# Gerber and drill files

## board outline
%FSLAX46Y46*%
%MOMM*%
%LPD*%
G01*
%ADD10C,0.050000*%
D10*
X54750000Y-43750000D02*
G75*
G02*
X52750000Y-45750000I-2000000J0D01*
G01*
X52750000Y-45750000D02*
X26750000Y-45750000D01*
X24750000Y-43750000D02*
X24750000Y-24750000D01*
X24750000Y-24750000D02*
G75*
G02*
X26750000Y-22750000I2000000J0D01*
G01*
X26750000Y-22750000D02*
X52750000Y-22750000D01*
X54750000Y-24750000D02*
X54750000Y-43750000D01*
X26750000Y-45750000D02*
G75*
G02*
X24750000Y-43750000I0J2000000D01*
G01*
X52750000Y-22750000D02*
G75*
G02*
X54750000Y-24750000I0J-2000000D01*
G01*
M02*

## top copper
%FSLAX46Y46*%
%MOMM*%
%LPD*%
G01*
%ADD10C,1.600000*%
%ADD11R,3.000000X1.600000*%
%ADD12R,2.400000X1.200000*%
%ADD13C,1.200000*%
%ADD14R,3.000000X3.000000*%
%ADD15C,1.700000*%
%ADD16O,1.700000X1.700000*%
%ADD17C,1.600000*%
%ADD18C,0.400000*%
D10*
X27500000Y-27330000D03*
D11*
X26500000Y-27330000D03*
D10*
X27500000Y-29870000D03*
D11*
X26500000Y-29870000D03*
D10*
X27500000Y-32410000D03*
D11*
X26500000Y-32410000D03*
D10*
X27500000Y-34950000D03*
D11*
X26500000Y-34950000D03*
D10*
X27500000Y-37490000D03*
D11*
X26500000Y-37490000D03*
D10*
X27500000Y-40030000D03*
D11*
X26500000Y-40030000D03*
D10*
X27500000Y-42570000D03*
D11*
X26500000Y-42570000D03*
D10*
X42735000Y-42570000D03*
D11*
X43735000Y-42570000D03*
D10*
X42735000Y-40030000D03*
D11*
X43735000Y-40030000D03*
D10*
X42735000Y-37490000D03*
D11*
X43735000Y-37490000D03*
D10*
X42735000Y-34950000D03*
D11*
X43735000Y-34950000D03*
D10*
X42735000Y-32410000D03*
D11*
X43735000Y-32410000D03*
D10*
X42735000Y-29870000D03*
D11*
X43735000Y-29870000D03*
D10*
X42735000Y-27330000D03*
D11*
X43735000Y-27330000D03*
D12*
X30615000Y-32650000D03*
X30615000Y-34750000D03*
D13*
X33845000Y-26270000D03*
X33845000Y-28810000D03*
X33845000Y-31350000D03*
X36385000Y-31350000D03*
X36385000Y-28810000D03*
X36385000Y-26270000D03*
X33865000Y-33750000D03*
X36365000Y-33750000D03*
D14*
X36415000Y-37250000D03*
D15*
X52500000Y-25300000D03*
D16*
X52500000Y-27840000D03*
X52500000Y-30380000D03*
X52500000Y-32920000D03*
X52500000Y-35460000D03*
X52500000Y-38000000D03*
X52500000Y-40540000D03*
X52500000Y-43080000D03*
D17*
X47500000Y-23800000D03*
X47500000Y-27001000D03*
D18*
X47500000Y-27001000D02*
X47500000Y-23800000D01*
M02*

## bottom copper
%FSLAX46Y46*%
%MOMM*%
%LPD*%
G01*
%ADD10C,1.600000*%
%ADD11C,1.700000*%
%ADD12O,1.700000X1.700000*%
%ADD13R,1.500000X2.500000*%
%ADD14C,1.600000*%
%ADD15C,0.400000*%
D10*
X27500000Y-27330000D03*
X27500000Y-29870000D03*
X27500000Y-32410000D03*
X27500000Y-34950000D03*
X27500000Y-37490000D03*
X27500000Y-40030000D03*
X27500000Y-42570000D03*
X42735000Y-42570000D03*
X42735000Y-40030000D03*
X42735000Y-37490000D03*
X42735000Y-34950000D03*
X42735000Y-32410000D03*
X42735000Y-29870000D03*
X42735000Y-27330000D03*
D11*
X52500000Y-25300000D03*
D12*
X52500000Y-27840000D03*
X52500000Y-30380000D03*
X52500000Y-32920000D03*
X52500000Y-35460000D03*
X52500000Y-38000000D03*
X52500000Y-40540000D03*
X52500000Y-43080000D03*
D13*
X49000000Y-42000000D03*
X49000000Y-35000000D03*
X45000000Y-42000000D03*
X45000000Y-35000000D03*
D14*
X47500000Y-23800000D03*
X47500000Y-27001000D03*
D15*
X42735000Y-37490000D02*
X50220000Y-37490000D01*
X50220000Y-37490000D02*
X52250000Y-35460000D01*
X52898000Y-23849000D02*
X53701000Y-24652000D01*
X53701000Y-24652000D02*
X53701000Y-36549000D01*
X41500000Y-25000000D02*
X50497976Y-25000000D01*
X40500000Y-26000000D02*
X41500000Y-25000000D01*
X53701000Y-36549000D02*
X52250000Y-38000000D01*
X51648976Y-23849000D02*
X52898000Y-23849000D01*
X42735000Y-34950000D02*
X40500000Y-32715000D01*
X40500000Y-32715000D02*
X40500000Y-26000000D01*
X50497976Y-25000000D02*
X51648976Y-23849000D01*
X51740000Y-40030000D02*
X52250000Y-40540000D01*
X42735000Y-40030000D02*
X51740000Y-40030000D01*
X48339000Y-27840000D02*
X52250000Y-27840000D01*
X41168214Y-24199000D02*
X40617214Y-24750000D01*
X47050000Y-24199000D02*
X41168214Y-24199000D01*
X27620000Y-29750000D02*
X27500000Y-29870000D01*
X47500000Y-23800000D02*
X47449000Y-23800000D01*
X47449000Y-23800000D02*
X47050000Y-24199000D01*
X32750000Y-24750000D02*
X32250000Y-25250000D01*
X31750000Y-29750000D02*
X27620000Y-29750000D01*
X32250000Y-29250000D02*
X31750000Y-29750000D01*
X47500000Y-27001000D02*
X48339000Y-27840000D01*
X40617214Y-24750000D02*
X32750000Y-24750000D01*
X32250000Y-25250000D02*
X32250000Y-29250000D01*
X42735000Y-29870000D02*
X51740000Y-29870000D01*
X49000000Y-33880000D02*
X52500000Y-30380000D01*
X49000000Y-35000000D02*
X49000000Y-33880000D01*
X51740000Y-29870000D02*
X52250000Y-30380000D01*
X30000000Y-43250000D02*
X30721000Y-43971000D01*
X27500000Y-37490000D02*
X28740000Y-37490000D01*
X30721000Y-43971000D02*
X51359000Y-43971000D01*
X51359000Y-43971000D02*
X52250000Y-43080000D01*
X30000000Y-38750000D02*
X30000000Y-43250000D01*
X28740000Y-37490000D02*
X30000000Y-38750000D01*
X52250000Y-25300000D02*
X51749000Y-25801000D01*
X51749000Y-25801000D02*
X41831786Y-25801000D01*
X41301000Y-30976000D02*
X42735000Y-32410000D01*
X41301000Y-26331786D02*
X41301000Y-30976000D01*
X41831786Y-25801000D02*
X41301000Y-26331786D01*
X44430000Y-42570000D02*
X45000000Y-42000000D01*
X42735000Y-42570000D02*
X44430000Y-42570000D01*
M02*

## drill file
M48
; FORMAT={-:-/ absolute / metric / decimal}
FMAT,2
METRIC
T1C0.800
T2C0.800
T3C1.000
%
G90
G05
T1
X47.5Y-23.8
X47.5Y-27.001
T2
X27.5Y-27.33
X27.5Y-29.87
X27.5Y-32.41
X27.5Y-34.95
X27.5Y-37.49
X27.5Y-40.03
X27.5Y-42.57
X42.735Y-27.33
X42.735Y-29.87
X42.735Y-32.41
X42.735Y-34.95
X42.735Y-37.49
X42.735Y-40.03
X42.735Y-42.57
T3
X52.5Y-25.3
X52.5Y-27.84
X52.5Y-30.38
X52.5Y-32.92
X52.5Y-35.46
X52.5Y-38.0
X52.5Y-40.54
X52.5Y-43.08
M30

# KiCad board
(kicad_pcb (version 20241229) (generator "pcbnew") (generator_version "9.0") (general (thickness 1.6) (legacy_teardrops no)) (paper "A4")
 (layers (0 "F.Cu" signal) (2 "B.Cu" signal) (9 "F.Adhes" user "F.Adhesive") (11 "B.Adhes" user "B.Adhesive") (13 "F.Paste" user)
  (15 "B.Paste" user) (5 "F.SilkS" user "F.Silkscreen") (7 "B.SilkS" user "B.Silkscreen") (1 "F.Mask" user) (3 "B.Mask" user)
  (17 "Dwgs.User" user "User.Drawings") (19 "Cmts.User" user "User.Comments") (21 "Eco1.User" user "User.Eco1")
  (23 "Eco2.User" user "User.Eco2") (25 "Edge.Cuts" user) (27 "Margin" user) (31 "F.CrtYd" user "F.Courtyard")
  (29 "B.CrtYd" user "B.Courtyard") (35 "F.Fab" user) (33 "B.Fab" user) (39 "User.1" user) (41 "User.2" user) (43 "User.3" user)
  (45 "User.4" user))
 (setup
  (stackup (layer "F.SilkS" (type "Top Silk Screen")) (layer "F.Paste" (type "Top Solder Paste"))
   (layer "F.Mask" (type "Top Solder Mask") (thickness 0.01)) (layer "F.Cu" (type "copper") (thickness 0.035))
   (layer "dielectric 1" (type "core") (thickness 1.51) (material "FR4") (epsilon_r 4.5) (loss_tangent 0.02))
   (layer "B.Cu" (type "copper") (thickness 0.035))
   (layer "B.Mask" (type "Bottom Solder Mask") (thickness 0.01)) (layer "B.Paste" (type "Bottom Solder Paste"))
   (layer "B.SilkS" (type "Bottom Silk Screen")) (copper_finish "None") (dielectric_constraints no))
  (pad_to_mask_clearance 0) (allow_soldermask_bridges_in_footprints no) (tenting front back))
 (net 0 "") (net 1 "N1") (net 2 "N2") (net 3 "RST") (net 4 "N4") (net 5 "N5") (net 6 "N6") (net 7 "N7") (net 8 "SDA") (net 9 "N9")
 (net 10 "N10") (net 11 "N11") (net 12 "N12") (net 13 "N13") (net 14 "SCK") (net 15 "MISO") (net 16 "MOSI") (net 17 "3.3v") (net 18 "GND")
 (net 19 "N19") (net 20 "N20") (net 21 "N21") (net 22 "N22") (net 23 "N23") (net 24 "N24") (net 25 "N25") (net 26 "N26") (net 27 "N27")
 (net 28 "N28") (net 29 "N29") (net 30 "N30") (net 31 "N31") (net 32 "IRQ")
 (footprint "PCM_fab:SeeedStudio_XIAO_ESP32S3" (layer "F.Cu") (at 35.115 34.95)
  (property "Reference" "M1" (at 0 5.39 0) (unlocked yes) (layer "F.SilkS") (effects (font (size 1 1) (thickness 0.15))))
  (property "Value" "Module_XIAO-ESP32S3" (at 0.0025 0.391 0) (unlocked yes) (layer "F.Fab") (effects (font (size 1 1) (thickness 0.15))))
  (pad "1" thru_hole circle (at -7.615 -7.62) (size 1.6 1.6) (drill 0.8) (layers "*.Cu" "*.Mask") (remove_unused_layers no) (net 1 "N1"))
  (pad "1" smd rect (at -7.615 -7.62) (size 3 1.6) (drill (offset -1 0)) (layers "F.Cu" "F.Mask" "F.Paste") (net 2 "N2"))
  (pad "2" thru_hole circle (at -7.615 -5.08) (size 1.6 1.6) (drill 0.8) (layers "*.Cu" "*.Mask") (remove_unused_layers no) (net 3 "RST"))
  (pad "2" smd rect (at -7.615 -5.08) (size 3 1.6) (drill (offset -1 0)) (layers "F.Cu" "F.Mask" "F.Paste") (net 3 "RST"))
  (pad "3" thru_hole circle (at -7.615 -2.54) (size 1.6 1.6) (drill 0.8) (layers "*.Cu" "*.Mask") (remove_unused_layers no) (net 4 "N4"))
  (pad "3" smd rect (at -7.615 -2.54) (size 3 1.6) (drill (offset -1 0)) (layers "F.Cu" "F.Mask" "F.Paste") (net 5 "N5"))
  (pad "4" thru_hole circle (at -7.615 0) (size 1.6 1.6) (drill 0.8) (layers "*.Cu" "*.Mask") (remove_unused_layers no) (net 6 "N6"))
  (pad "4" smd rect (at -7.615 0) (size 3 1.6) (drill (offset -1 0)) (layers "F.Cu" "F.Mask" "F.Paste") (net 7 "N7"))
  (pad "5" thru_hole circle (at -7.615 2.54) (size 1.6 1.6) (drill 0.8) (layers "*.Cu" "*.Mask") (remove_unused_layers no) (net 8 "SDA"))
  (pad "5" smd rect (at -7.615 2.54) (size 3 1.6) (drill (offset -1 0)) (layers "F.Cu" "F.Mask" "F.Paste") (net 8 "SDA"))
  (pad "6" thru_hole circle (at -7.615 5.08) (size 1.6 1.6) (drill 0.8) (layers "*.Cu" "*.Mask") (remove_unused_layers no) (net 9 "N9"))
  (pad "6" smd rect (at -7.615 5.08) (size 3 1.6) (drill (offset -1 0)) (layers "F.Cu" "F.Mask" "F.Paste") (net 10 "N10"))
  (pad "7" thru_hole circle (at -7.615 7.62) (size 1.6 1.6) (drill 0.8) (layers "*.Cu" "*.Mask") (remove_unused_layers no) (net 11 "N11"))
  (pad "7" smd rect (at -7.615 7.62) (size 3 1.6) (drill (offset -1 0)) (layers "F.Cu" "F.Mask" "F.Paste") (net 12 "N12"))
  (pad "8" thru_hole circle (at 7.62 7.62) (size 1.6 1.6) (drill 0.8) (layers "*.Cu" "*.Mask") (remove_unused_layers no) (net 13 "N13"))
  (pad "8" smd rect (at 7.62 7.62) (size 3 1.6) (drill (offset 1 0)) (layers "F.Cu" "F.Mask" "F.Paste") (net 13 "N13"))
  (pad "9" thru_hole circle (at 7.62 5.08) (size 1.6 1.6) (drill 0.8) (layers "*.Cu" "*.Mask") (remove_unused_layers no) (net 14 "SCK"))
  (pad "9" smd rect (at 7.62 5.08) (size 3 1.6) (drill (offset 1 0)) (layers "F.Cu" "F.Mask" "F.Paste") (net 14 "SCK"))
  (pad "10" thru_hole circle (at 7.62 2.54) (size 1.6 1.6) (drill 0.8) (layers "*.Cu" "*.Mask") (remove_unused_layers no) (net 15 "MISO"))
  (pad "10" smd rect (at 7.62 2.54) (size 3 1.6) (drill (offset 1 0)) (layers "F.Cu" "F.Mask" "F.Paste") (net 15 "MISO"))
  (pad "11" thru_hole circle (at 7.62 0) (size 1.6 1.6) (drill 0.8) (layers "*.Cu" "*.Mask") (remove_unused_layers no) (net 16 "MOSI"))
  (pad "11" smd rect (at 7.62 0) (size 3 1.6) (drill (offset 1 0)) (layers "F.Cu" "F.Mask" "F.Paste") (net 16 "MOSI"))
  (pad "12" thru_hole circle (at 7.62 -2.54) (size 1.6 1.6) (drill 0.8) (layers "*.Cu" "*.Mask") (remove_unused_layers no) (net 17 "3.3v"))
  (pad "12" smd rect (at 7.62 -2.54) (size 3 1.6) (drill (offset 1 0)) (layers "F.Cu" "F.Mask" "F.Paste") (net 17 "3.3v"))
  (pad "13" thru_hole circle (at 7.62 -5.08) (size 1.6 1.6) (drill 0.8) (layers "*.Cu" "*.Mask") (remove_unused_layers no) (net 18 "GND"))
  (pad "13" smd rect (at 7.62 -5.08) (size 3 1.6) (drill (offset 1 0)) (layers "F.Cu" "F.Mask" "F.Paste") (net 18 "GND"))
  (pad "14" thru_hole circle (at 7.62 -7.62) (size 1.6 1.6) (drill 0.8) (layers "*.Cu" "*.Mask") (remove_unused_layers no) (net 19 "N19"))
  (pad "14" smd rect (at 7.62 -7.62) (size 3 1.6) (drill (offset 1 0)) (layers "F.Cu" "F.Mask" "F.Paste") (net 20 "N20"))
  (pad "15" smd rect (at -4.5 -2.3) (size 2.4 1.2) (layers "F.Cu" "F.Mask" "F.Paste") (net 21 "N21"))
  (pad "16" smd rect (at -4.5 -0.2) (size 2.4 1.2) (layers "F.Cu" "F.Mask" "F.Paste") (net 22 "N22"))
  (pad "17" smd circle (at -1.27 -8.68) (size 1.2 1.2) (layers "F.Cu" "F.Mask" "F.Paste") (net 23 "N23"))
  (pad "18" smd circle (at -1.27 -6.14) (size 1.2 1.2) (layers "F.Cu" "F.Mask" "F.Paste") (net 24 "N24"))
  (pad "19" smd circle (at -1.27 -3.6) (size 1.2 1.2) (layers "F.Cu" "F.Mask" "F.Paste") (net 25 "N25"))
  (pad "20" smd circle (at 1.27 -3.6) (size 1.2 1.2) (layers "F.Cu" "F.Mask" "F.Paste") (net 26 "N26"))
  (pad "21" smd circle (at 1.27 -6.14) (size 1.2 1.2) (layers "F.Cu" "F.Mask" "F.Paste") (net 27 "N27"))
  (pad "22" smd circle (at 1.27 -8.68) (size 1.2 1.2) (layers "F.Cu" "F.Mask" "F.Paste") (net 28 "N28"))
  (pad "23" smd circle (at -1.25 -1.2) (size 1.2 1.2) (layers "F.Cu" "F.Mask" "F.Paste") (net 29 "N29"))
  (pad "24" smd circle (at 1.25 -1.2) (size 1.2 1.2) (layers "F.Cu" "F.Mask" "F.Paste") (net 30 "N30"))
  (pad "25" smd rect (at 1.3 2.3) (size 3 3) (layers "F.Cu" "F.Mask" "F.Paste") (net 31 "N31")))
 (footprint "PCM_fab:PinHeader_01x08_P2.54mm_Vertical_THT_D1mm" (layer "B.Cu") (at 52.5 25.3 180)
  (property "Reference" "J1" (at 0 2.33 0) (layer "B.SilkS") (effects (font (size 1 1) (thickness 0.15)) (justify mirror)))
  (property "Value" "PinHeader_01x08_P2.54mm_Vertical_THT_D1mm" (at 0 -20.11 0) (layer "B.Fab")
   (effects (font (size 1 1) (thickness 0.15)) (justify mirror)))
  (pad "1" thru_hole circle (at 0 0 180) (size 1.7 1.7) (drill 1) (layers "*.Cu" "*.Mask") (remove_unused_layers no) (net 17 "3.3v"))
  (pad "2" thru_hole oval (at 0 -2.54 180) (size 1.7 1.7) (drill 1) (layers "*.Cu" "*.Mask") (remove_unused_layers no) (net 3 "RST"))
  (pad "3" thru_hole oval (at 0 -5.08 180) (size 1.7 1.7) (drill 1) (layers "*.Cu" "*.Mask") (remove_unused_layers no) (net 18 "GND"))
  (pad "4" thru_hole oval (at 0 -7.62 180) (size 1.7 1.7) (drill 1) (layers "*.Cu" "*.Mask") (remove_unused_layers no) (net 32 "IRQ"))
  (pad "5" thru_hole oval (at 0 -10.16 180) (size 1.7 1.7) (drill 1) (layers "*.Cu" "*.Mask") (remove_unused_layers no) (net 15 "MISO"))
  (pad "6" thru_hole oval (at 0 -12.7 180) (size 1.7 1.7) (drill 1) (layers "*.Cu" "*.Mask") (remove_unused_layers no) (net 16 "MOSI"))
  (pad "7" thru_hole oval (at 0 -15.24 180) (size 1.7 1.7) (drill 1) (layers "*.Cu" "*.Mask") (remove_unused_layers no) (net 14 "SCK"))
  (pad "8" thru_hole oval (at 0 -17.78 180) (size 1.7 1.7) (drill 1) (layers "*.Cu" "*.Mask") (remove_unused_layers no) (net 8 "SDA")))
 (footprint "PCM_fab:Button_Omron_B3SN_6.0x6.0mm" (layer "B.Cu") (at 47 38.5 90)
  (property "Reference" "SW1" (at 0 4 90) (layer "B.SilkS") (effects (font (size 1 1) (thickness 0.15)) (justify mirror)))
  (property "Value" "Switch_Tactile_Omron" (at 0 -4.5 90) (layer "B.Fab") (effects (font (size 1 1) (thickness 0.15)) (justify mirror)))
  (pad "1" smd rect (at -3.5 2 90) (size 2.5 1.5) (layers "B.Cu" "B.Mask" "B.Paste") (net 18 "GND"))
  (pad "1" smd rect (at 3.5 2 90) (size 2.5 1.5) (layers "B.Cu" "B.Mask" "B.Paste") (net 18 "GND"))
  (pad "2" smd rect (at -3.5 -2 90) (size 2.5 1.5) (layers "B.Cu" "B.Mask" "B.Paste") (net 13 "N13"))
  (pad "2" smd rect (at 3.5 -2 90) (size 2.5 1.5) (layers "B.Cu" "B.Mask" "B.Paste") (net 13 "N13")))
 (gr_arc (start 54.75 43.75) (mid 54.164214 45.164214) (end 52.75 45.75) (stroke (width 0.05) (type default)) (layer "Edge.Cuts"))
 (gr_line (start 52.75 45.75) (end 26.75 45.75) (stroke (width 0.05) (type default)) (layer "Edge.Cuts"))
 (gr_line (start 24.75 43.75) (end 24.75 24.75) (stroke (width 0.05) (type default)) (layer "Edge.Cuts"))
 (gr_arc (start 24.75 24.75) (mid 25.335786 23.335786) (end 26.75 22.75) (stroke (width 0.05) (type default)) (layer "Edge.Cuts"))
 (gr_line (start 26.75 22.75) (end 52.75 22.75) (stroke (width 0.05) (type default)) (layer "Edge.Cuts"))
 (gr_line (start 54.75 24.75) (end 54.75 43.75) (stroke (width 0.05) (type default)) (layer "Edge.Cuts"))
 (gr_arc (start 26.75 45.75) (mid 25.335786 45.164214) (end 24.75 43.75) (stroke (width 0.05) (type default)) (layer "Edge.Cuts"))
 (gr_arc (start 52.75 22.75) (mid 54.164214 23.335786) (end 54.75 24.75) (stroke (width 0.05) (type default)) (layer "Edge.Cuts"))
 (segment (start 42.735 37.49) (end 50.22 37.49) (width 0.4) (layer "B.Cu") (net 15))
 (segment (start 50.22 37.49) (end 52.25 35.46) (width 0.4) (layer "B.Cu") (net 15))
 (segment (start 52.898 23.849) (end 53.701 24.652) (width 0.4) (layer "B.Cu") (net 16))
 (segment (start 53.701 24.652) (end 53.701 36.549) (width 0.4) (layer "B.Cu") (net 16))
 (segment (start 41.5 25) (end 50.497976 25) (width 0.4) (layer "B.Cu") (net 16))
 (segment (start 40.5 26) (end 41.5 25) (width 0.4) (layer "B.Cu") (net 16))
 (segment (start 53.701 36.549) (end 52.25 38) (width 0.4) (layer "B.Cu") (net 16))
 (segment (start 51.648976 23.849) (end 52.898 23.849) (width 0.4) (layer "B.Cu") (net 16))
 (segment (start 42.735 34.95) (end 40.5 32.715) (width 0.4) (layer "B.Cu") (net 16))
 (segment (start 40.5 32.715) (end 40.5 26) (width 0.4) (layer "B.Cu") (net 16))
 (segment (start 50.497976 25) (end 51.648976 23.849) (width 0.4) (layer "B.Cu") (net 16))
 (segment (start 51.74 40.03) (end 52.25 40.54) (width 0.4) (layer "B.Cu") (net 14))
 (segment (start 42.735 40.03) (end 51.74 40.03) (width 0.4) (layer "B.Cu") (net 14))
 (segment (start 47.5 27.001) (end 47.5 23.8) (width 0.4) (layer "F.Cu") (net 3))
 (via (at 47.5 23.8) (size 1.6) (drill 0.8) (layers "F.Cu" "B.Cu") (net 3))
 (via (at 47.5 27.001) (size 1.6) (drill 0.8) (layers "F.Cu" "B.Cu") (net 3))
 (segment (start 48.339 27.84) (end 52.25 27.84) (width 0.4) (layer "B.Cu") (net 3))
 (segment (start 41.168214 24.199) (end 40.617214 24.75) (width 0.4) (layer "B.Cu") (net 3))
 (segment (start 47.05 24.199) (end 41.168214 24.199) (width 0.4) (layer "B.Cu") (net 3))
 (segment (start 27.62 29.75) (end 27.5 29.87) (width 0.4) (layer "B.Cu") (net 3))
 (segment (start 47.5 23.8) (end 47.449 23.8) (width 0.4) (layer "B.Cu") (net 3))
 (segment (start 47.449 23.8) (end 47.05 24.199) (width 0.4) (layer "B.Cu") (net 3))
 (segment (start 32.75 24.75) (end 32.25 25.25) (width 0.4) (layer "B.Cu") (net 3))
 (segment (start 31.75 29.75) (end 27.62 29.75) (width 0.4) (layer "B.Cu") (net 3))
 (segment (start 32.25 29.25) (end 31.75 29.75) (width 0.4) (layer "B.Cu") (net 3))
 (segment (start 47.5 27.001) (end 48.339 27.84) (width 0.4) (layer "B.Cu") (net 3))
 (segment (start 40.617214 24.75) (end 32.75 24.75) (width 0.4) (layer "B.Cu") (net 3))
 (segment (start 32.25 25.25) (end 32.25 29.25) (width 0.4) (layer "B.Cu") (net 3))
 (segment (start 42.735 29.87) (end 51.74 29.87) (width 0.4) (layer "B.Cu") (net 18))
 (segment (start 49 33.88) (end 52.5 30.38) (width 0.4) (layer "B.Cu") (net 18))
 (segment (start 49 35) (end 49 33.88) (width 0.4) (layer "B.Cu") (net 18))
 (segment (start 51.74 29.87) (end 52.25 30.38) (width 0.4) (layer "B.Cu") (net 18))
 (segment (start 30 43.25) (end 30.721 43.971) (width 0.4) (layer "B.Cu") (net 8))
 (segment (start 27.5 37.49) (end 28.74 37.49) (width 0.4) (layer "B.Cu") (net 8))
 (segment (start 30.721 43.971) (end 51.359 43.971) (width 0.4) (layer "B.Cu") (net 8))
 (segment (start 51.359 43.971) (end 52.25 43.08) (width 0.4) (layer "B.Cu") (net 8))
 (segment (start 30 38.75) (end 30 43.25) (width 0.4) (layer "B.Cu") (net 8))
 (segment (start 28.74 37.49) (end 30 38.75) (width 0.4) (layer "B.Cu") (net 8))
 (segment (start 52.25 25.3) (end 51.749 25.801) (width 0.4) (layer "B.Cu") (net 17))
 (segment (start 51.749 25.801) (end 41.831786 25.801) (width 0.4) (layer "B.Cu") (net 17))
 (segment (start 41.301 30.976) (end 42.735 32.41) (width 0.4) (layer "B.Cu") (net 17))
 (segment (start 41.301 26.331786) (end 41.301 30.976) (width 0.4) (layer "B.Cu") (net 17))
 (segment (start 41.831786 25.801) (end 41.301 26.331786) (width 0.4) (layer "B.Cu") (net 17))
 (segment (start 44.43 42.57) (end 45 42) (width 0.4) (layer "B.Cu") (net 13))
 (segment (start 42.735 42.57) (end 44.43 42.57) (width 0.4) (layer "B.Cu") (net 13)))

